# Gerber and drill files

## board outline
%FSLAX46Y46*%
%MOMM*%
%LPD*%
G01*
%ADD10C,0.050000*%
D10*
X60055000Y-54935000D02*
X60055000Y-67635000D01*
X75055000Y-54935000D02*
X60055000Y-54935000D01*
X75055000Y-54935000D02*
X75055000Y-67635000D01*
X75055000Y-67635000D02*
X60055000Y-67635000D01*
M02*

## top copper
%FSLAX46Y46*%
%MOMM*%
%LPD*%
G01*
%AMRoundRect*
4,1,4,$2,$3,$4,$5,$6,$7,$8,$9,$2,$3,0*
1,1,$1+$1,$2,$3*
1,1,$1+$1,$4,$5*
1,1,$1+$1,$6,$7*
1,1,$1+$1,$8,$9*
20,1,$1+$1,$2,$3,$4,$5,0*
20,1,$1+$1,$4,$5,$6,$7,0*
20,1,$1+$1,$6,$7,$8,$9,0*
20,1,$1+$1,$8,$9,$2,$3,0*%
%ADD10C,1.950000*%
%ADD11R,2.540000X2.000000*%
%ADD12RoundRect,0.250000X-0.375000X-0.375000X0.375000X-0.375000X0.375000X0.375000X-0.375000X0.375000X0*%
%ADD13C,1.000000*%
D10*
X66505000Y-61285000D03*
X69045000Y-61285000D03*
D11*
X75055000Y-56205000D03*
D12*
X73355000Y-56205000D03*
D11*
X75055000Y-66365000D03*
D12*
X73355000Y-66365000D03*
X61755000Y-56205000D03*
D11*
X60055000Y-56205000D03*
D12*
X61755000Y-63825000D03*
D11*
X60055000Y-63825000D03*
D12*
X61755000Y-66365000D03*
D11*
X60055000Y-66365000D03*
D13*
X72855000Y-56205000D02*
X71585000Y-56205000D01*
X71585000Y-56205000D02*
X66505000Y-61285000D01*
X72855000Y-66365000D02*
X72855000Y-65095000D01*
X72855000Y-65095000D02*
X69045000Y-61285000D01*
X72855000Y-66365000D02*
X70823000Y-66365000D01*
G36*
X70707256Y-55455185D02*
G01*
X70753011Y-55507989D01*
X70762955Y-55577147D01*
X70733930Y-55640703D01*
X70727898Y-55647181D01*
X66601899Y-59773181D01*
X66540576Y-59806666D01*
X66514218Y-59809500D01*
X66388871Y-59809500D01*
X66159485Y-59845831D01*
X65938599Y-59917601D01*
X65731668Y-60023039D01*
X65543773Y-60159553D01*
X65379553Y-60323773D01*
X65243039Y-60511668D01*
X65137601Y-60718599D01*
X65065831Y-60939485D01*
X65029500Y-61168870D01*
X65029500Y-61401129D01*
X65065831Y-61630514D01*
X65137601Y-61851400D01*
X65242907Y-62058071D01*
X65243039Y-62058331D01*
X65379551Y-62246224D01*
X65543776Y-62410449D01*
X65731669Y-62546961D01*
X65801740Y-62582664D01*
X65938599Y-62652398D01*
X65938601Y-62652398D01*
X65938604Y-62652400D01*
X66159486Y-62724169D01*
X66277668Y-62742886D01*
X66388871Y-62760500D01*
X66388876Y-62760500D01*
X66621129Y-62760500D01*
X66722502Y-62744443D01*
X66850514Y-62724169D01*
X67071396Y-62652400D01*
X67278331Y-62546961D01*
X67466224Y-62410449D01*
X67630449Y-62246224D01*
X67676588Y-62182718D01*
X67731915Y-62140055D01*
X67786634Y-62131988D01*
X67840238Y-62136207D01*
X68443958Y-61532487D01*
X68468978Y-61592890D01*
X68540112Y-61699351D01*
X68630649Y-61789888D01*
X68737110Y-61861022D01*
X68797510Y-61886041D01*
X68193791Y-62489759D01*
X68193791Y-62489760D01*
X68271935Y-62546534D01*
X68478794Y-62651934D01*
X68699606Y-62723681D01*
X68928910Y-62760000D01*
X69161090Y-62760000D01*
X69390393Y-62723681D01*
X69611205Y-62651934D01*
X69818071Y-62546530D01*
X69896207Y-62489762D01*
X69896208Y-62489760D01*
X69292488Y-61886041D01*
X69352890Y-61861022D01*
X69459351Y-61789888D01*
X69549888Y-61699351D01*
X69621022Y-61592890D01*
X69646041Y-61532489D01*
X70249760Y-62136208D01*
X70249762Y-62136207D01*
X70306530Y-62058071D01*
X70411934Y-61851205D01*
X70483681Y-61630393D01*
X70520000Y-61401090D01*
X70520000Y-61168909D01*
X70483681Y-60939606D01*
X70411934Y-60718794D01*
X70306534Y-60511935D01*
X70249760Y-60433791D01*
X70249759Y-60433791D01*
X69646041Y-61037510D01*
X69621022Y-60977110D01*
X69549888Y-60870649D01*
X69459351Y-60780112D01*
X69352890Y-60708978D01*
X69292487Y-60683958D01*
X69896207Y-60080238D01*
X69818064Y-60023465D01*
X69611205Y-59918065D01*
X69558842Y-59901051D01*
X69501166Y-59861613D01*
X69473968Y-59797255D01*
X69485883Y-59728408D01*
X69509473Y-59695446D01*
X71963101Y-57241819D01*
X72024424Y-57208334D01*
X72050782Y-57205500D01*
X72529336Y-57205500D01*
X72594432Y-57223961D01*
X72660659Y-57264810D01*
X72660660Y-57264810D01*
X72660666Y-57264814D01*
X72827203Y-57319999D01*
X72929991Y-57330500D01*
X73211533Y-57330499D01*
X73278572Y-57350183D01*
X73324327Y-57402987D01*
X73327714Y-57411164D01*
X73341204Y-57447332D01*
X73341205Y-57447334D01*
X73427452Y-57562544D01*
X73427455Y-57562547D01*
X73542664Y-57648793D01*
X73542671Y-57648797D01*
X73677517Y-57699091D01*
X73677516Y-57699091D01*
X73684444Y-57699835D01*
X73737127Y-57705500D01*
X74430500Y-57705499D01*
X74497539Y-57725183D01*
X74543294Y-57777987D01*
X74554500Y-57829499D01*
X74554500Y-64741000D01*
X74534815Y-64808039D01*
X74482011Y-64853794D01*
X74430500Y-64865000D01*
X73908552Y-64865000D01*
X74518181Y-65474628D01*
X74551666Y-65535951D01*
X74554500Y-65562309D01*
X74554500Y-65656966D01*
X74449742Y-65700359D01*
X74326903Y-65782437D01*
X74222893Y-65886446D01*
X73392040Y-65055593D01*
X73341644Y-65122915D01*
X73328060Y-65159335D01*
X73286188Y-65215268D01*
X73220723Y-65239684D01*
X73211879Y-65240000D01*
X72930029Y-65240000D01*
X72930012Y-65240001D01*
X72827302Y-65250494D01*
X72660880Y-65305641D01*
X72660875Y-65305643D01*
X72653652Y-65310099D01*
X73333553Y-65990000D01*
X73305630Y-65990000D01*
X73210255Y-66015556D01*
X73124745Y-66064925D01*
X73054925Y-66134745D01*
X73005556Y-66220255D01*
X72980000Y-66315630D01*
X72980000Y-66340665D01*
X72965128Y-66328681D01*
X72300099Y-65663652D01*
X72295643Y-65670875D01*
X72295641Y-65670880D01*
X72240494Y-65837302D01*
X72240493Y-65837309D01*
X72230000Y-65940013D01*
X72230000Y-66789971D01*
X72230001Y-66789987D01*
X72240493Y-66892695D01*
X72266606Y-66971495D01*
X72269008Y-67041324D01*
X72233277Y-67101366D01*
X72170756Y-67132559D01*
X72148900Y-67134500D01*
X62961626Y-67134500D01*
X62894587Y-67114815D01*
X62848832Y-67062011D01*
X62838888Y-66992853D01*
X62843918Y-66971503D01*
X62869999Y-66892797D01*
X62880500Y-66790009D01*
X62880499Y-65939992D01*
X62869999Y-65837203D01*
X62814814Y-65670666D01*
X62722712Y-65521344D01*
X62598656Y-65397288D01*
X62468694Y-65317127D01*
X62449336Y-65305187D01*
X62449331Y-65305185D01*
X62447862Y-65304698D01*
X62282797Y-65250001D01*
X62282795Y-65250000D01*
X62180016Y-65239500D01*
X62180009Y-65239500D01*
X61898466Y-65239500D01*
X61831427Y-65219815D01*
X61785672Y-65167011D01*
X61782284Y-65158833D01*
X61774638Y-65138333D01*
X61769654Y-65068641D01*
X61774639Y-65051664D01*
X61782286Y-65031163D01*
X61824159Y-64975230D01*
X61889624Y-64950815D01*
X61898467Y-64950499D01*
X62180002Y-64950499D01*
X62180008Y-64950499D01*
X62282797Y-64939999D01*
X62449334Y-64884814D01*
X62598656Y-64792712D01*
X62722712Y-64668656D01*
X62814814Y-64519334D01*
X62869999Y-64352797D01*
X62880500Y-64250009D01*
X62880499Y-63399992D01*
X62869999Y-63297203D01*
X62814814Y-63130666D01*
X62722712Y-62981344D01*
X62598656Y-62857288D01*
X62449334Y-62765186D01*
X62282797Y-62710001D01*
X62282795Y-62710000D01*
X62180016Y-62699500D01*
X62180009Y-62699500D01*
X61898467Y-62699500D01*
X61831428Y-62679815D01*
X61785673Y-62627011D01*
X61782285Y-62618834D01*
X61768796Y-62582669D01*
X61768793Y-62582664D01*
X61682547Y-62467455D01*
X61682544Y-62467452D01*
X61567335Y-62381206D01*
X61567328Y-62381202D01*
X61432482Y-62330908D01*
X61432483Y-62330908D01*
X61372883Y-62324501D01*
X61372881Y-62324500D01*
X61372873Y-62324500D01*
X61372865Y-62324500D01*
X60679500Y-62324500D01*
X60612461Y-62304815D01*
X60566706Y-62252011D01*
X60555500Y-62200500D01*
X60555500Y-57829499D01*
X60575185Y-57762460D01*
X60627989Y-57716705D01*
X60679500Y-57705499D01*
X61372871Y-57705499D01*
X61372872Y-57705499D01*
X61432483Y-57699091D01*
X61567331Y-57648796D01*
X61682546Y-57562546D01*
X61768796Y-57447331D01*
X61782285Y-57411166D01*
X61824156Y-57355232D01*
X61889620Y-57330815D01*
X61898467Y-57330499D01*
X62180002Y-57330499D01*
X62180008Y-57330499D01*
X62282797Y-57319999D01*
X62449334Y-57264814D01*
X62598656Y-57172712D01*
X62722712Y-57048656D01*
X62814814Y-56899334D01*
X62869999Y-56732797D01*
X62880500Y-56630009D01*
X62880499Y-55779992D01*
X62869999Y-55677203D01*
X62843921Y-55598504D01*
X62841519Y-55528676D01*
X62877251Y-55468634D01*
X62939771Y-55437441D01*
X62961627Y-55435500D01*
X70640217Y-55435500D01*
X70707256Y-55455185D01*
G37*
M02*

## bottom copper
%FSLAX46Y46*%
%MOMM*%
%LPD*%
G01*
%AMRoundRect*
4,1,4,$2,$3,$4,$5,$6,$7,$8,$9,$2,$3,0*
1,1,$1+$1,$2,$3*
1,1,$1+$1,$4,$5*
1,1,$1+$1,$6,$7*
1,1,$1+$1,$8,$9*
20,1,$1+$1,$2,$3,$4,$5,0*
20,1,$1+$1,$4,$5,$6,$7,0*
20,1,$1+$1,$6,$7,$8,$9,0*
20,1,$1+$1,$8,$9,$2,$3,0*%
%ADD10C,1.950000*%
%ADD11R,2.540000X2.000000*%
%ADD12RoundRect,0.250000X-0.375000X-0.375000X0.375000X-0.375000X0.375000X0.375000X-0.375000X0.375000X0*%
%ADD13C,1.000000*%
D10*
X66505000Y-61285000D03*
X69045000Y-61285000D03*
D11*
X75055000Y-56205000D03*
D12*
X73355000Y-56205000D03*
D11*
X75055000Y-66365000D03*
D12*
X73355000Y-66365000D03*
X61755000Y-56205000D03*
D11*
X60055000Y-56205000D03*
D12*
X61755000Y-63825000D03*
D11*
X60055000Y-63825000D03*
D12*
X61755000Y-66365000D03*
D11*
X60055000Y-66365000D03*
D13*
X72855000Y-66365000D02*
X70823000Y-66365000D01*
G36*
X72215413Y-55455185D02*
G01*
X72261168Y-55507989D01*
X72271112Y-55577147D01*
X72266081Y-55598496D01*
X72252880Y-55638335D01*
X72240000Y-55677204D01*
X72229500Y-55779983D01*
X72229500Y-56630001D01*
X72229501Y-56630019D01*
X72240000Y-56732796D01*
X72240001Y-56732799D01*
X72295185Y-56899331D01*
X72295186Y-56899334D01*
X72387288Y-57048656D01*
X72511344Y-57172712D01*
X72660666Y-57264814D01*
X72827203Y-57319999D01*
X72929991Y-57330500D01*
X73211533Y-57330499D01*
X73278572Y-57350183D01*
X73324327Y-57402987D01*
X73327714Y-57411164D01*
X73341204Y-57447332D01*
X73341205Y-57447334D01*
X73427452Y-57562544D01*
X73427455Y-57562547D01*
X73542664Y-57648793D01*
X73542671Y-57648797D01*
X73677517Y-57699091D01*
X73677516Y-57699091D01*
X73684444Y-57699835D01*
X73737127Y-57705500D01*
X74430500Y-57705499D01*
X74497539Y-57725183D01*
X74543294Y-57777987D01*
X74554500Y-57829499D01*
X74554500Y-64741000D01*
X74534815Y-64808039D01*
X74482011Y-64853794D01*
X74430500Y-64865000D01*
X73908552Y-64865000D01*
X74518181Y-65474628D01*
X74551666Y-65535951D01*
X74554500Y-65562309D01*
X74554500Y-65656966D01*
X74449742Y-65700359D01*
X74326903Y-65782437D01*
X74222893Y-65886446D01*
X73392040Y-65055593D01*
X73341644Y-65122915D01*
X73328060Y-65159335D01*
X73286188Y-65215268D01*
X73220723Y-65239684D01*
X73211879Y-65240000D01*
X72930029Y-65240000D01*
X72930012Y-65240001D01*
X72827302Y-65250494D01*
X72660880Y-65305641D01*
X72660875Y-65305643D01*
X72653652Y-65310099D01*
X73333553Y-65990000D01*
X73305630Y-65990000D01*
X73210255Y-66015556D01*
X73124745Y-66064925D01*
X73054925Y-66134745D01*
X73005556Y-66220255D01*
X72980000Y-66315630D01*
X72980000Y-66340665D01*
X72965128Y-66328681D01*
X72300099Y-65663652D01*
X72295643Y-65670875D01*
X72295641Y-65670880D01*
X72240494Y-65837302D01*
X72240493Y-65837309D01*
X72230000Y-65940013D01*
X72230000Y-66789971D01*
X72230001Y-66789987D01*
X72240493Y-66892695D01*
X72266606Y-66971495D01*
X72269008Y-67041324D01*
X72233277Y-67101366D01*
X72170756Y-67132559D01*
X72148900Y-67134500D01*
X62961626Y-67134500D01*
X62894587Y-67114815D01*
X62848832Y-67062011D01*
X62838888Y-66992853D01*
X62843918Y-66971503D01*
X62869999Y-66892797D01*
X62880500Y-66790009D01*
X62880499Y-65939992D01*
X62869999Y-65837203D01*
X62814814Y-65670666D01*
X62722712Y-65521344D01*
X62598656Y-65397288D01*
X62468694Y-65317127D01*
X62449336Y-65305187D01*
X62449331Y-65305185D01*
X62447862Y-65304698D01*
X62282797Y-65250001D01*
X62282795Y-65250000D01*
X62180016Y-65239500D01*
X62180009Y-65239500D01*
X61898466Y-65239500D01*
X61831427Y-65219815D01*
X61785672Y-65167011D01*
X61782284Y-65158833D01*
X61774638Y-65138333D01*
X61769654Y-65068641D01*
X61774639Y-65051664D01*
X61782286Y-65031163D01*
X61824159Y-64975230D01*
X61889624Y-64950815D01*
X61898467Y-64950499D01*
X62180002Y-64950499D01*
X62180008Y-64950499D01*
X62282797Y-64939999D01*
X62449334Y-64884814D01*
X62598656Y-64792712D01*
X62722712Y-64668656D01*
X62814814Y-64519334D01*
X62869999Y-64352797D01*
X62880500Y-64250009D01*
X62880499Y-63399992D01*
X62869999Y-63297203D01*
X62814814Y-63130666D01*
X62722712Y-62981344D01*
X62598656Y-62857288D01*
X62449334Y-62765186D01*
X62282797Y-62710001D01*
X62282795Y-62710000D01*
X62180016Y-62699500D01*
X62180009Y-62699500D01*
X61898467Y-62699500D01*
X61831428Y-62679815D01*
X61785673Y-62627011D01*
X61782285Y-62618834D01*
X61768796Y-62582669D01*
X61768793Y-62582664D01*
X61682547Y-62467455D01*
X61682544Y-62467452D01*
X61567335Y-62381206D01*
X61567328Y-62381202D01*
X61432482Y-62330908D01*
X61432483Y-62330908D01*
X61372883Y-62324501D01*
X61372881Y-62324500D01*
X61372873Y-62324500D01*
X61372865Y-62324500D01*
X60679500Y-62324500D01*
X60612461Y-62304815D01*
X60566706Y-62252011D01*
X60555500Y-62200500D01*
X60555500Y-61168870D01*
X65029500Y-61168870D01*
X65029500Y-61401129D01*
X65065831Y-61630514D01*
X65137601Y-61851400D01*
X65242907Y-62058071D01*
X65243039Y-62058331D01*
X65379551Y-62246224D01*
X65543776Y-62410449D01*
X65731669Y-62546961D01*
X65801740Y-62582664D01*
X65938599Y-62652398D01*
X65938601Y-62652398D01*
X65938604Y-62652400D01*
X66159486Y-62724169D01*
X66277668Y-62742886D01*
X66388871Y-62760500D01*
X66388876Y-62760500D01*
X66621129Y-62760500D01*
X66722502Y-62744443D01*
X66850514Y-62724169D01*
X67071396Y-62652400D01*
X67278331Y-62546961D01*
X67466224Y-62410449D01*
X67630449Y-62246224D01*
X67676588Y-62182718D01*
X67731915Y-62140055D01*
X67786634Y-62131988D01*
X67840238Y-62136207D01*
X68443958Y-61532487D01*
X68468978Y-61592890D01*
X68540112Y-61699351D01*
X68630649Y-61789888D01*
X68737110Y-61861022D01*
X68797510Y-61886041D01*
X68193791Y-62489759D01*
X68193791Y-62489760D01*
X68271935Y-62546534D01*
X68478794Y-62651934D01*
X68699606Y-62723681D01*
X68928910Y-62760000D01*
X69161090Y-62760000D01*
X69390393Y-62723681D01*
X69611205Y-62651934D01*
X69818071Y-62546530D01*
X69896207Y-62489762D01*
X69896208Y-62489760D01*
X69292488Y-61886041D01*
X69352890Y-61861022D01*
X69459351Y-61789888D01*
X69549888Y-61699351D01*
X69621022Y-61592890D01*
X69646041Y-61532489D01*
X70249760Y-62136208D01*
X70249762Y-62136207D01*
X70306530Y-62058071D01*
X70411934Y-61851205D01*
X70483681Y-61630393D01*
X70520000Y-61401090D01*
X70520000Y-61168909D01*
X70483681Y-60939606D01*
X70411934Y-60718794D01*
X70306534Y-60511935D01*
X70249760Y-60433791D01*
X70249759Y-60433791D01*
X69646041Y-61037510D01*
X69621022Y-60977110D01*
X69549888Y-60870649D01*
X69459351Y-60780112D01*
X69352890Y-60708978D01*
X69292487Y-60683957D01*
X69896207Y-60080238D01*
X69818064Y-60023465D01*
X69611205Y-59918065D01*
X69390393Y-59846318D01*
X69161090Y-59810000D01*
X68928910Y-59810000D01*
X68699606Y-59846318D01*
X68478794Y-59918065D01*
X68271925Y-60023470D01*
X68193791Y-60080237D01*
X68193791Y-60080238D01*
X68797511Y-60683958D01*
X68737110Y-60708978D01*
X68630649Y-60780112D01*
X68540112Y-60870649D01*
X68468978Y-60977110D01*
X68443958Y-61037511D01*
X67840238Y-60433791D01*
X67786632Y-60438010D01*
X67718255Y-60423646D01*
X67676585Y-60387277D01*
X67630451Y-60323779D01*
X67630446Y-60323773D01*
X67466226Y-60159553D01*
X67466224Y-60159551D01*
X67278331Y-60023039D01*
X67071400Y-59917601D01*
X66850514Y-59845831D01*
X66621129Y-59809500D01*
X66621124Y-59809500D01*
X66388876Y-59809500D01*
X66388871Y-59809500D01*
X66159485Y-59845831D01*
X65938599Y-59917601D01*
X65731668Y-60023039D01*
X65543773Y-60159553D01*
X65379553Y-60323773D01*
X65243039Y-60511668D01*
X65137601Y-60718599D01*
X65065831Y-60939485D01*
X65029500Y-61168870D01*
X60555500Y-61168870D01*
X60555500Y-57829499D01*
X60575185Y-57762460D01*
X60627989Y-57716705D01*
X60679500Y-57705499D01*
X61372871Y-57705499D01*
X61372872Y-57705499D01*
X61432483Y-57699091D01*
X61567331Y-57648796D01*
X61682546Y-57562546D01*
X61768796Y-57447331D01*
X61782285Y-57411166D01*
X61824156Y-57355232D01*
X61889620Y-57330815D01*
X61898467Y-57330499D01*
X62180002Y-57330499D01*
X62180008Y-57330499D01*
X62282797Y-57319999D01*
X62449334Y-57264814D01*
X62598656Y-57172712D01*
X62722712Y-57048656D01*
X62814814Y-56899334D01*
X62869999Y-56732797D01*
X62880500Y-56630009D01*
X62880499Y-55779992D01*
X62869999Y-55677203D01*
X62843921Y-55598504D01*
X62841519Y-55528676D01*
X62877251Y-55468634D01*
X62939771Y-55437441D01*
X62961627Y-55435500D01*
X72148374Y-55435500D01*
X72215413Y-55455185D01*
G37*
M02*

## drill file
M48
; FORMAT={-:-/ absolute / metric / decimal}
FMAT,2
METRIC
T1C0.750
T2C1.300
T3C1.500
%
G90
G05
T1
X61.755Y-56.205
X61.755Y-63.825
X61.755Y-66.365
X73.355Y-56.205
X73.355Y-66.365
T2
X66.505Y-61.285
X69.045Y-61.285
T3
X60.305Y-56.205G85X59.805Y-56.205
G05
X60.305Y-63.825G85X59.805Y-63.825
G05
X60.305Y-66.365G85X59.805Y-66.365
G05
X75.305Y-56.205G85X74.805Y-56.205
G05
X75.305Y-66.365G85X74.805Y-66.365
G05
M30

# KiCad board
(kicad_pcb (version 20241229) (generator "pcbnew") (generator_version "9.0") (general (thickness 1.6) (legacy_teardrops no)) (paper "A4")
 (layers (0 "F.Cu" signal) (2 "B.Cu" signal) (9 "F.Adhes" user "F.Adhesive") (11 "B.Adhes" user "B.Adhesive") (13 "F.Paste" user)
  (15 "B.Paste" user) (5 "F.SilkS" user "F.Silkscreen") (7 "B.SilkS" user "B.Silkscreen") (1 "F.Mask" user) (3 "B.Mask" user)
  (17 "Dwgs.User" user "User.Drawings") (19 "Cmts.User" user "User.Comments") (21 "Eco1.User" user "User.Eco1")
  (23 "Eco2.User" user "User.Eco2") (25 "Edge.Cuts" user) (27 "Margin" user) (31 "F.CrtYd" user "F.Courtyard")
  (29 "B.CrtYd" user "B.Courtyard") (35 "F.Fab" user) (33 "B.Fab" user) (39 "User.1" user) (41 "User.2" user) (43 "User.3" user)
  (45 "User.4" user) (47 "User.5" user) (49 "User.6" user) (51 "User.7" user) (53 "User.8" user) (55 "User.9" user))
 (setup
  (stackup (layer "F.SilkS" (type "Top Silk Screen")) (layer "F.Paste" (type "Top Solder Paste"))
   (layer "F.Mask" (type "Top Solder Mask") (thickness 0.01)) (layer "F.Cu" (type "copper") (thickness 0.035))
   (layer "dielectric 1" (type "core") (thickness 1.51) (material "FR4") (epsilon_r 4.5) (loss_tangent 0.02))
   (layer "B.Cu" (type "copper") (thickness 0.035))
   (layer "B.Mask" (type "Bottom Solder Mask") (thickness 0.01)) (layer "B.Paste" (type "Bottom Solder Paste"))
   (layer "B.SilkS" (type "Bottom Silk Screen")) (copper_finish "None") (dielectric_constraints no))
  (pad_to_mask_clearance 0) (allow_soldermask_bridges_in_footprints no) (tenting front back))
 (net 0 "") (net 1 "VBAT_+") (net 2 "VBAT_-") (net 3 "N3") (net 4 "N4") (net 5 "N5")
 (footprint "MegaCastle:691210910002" (layer "F.Cu") (at 67.775 61.285)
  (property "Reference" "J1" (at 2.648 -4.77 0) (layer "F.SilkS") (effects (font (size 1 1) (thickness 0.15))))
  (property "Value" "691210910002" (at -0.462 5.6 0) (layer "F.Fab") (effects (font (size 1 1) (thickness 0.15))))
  (pad "1" thru_hole circle (at -1.27 0) (size 1.95 1.95) (drill 1.3) (layers "*.Cu" "*.Mask") (remove_unused_layers no) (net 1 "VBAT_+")
   (solder_mask_margin 0.102))
  (pad "2" thru_hole circle (at 1.27 0) (size 1.95 1.95) (drill 1.3) (layers "*.Cu" "*.Mask") (remove_unused_layers no) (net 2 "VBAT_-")
   (solder_mask_margin 0.102)))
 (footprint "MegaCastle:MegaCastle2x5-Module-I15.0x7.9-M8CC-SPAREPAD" (layer "B.Cu") (at 67.555 61.285 180)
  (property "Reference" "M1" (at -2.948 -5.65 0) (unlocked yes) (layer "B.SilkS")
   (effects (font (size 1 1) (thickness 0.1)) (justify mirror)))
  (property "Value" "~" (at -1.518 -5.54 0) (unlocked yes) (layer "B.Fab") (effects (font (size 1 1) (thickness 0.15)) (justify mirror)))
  (fp_line (start 7.5 6.35) (end 7.5 -6.35) (stroke (width 0.05) (type default)) (layer "Edge.Cuts"))
  (fp_line (start -7.5 6.35) (end 7.5 6.35) (stroke (width 0.05) (type default)) (layer "Edge.Cuts"))
  (fp_line (start -7.5 6.35) (end -7.5 -6.35) (stroke (width 0.05) (type default)) (layer "Edge.Cuts"))
  (fp_line (start -7.5 -6.35) (end 7.5 -6.35) (stroke (width 0.05) (type default)) (layer "Edge.Cuts"))
  (pad "1" thru_hole rect (at -7.5 5.08 180) (size 2.54 2) (drill oval 2 1.5) (layers "*.Cu" "*.Mask") (remove_unused_layers no)
   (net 1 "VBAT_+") (thermal_bridge_angle 45))
  (pad "1" thru_hole roundrect (at -5.8 5.08) (size 1.25 1.25) (drill 0.75) (layers "*.Cu" "*.Mask") (remove_unused_layers no)
   (roundrect_rratio 0.2) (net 1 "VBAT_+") (thermal_bridge_angle 45))
  (pad "5" thru_hole rect (at -7.5 -5.08 180) (size 2.54 2) (drill oval 2 1.5) (layers "*.Cu" "*.Mask") (remove_unused_layers no)
   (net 2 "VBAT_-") (thermal_bridge_angle 45))
  (pad "5" thru_hole roundrect (at -5.8 -5.08) (size 1.25 1.25) (drill 0.75) (layers "*.Cu" "*.Mask") (remove_unused_layers no)
   (roundrect_rratio 0.2) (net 2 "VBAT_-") (thermal_bridge_angle 45))
  (pad "6" thru_hole roundrect (at 5.8 5.08) (size 1.25 1.25) (drill 0.75) (layers "*.Cu" "*.Mask") (remove_unused_layers no)
   (roundrect_rratio 0.2) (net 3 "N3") (thermal_bridge_angle 45))
  (pad "6" thru_hole rect (at 7.5 5.08 180) (size 2.54 2) (drill oval 2 1.5) (layers "*.Cu" "*.Mask") (remove_unused_layers no) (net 3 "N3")
   (thermal_bridge_angle 45))
  (pad "9" thru_hole roundrect (at 5.8 -2.54) (size 1.25 1.25) (drill 0.75) (layers "*.Cu" "*.Mask") (remove_unused_layers no)
   (roundrect_rratio 0.2) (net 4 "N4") (thermal_bridge_angle 45))
  (pad "9" thru_hole rect (at 7.5 -2.54 180) (size 2.54 2) (drill oval 2 1.5) (layers "*.Cu" "*.Mask") (remove_unused_layers no)
   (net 4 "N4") (thermal_bridge_angle 45))
  (pad "10" thru_hole roundrect (at 5.8 -5.08) (size 1.25 1.25) (drill 0.75) (layers "*.Cu" "*.Mask") (remove_unused_layers no)
   (roundrect_rratio 0.2) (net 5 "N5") (thermal_bridge_angle 45))
  (pad "10" thru_hole rect (at 7.5 -5.08 180) (size 2.54 2) (drill oval 2 1.5) (layers "*.Cu" "*.Mask") (remove_unused_layers no)
   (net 5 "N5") (thermal_bridge_angle 45))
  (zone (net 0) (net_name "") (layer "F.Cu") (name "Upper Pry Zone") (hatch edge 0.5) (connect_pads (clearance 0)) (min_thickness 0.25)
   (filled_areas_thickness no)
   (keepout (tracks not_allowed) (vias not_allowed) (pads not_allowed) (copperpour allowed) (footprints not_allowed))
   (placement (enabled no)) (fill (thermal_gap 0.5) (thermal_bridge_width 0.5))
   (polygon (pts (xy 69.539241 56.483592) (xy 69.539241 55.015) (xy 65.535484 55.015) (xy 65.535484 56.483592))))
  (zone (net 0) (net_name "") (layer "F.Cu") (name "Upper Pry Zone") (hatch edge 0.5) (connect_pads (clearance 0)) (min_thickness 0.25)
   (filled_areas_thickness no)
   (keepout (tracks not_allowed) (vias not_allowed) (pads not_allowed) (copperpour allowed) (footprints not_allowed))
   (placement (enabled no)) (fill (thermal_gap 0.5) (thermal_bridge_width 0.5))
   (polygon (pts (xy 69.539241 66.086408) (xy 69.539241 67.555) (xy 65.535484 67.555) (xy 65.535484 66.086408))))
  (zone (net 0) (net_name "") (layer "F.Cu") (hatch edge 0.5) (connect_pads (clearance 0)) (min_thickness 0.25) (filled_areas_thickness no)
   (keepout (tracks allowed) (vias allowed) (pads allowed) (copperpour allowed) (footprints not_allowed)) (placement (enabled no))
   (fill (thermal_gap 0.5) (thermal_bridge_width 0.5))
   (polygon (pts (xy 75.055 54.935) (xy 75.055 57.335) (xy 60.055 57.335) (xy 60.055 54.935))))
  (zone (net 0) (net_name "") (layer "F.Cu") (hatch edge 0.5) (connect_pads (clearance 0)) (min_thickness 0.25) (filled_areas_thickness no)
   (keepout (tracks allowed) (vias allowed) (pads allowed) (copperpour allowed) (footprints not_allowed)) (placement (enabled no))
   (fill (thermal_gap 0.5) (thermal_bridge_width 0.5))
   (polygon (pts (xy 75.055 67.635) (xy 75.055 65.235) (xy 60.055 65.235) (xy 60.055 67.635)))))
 (segment (start 72.855 56.205) (end 71.585 56.205) (width 1) (layer "F.Cu") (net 1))
 (segment (start 71.585 56.205) (end 66.505 61.285) (width 1) (layer "F.Cu") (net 1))
 (segment (start 72.855 66.365) (end 72.855 65.095) (width 1) (layer "F.Cu") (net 2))
 (segment (start 72.855 65.095) (end 69.045 61.285) (width 1) (layer "F.Cu") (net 2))
 (segment (start 72.855 66.365) (end 70.823 66.365) (width 1) (layer "F.Cu") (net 2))
 (segment (start 72.855 66.365) (end 70.823 66.365) (width 1) (layer "B.Cu") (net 2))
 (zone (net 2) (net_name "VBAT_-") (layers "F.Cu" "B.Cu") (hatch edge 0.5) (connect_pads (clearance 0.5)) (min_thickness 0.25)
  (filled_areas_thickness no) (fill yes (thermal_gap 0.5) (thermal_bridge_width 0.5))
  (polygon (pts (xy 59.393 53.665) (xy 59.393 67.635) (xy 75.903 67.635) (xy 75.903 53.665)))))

